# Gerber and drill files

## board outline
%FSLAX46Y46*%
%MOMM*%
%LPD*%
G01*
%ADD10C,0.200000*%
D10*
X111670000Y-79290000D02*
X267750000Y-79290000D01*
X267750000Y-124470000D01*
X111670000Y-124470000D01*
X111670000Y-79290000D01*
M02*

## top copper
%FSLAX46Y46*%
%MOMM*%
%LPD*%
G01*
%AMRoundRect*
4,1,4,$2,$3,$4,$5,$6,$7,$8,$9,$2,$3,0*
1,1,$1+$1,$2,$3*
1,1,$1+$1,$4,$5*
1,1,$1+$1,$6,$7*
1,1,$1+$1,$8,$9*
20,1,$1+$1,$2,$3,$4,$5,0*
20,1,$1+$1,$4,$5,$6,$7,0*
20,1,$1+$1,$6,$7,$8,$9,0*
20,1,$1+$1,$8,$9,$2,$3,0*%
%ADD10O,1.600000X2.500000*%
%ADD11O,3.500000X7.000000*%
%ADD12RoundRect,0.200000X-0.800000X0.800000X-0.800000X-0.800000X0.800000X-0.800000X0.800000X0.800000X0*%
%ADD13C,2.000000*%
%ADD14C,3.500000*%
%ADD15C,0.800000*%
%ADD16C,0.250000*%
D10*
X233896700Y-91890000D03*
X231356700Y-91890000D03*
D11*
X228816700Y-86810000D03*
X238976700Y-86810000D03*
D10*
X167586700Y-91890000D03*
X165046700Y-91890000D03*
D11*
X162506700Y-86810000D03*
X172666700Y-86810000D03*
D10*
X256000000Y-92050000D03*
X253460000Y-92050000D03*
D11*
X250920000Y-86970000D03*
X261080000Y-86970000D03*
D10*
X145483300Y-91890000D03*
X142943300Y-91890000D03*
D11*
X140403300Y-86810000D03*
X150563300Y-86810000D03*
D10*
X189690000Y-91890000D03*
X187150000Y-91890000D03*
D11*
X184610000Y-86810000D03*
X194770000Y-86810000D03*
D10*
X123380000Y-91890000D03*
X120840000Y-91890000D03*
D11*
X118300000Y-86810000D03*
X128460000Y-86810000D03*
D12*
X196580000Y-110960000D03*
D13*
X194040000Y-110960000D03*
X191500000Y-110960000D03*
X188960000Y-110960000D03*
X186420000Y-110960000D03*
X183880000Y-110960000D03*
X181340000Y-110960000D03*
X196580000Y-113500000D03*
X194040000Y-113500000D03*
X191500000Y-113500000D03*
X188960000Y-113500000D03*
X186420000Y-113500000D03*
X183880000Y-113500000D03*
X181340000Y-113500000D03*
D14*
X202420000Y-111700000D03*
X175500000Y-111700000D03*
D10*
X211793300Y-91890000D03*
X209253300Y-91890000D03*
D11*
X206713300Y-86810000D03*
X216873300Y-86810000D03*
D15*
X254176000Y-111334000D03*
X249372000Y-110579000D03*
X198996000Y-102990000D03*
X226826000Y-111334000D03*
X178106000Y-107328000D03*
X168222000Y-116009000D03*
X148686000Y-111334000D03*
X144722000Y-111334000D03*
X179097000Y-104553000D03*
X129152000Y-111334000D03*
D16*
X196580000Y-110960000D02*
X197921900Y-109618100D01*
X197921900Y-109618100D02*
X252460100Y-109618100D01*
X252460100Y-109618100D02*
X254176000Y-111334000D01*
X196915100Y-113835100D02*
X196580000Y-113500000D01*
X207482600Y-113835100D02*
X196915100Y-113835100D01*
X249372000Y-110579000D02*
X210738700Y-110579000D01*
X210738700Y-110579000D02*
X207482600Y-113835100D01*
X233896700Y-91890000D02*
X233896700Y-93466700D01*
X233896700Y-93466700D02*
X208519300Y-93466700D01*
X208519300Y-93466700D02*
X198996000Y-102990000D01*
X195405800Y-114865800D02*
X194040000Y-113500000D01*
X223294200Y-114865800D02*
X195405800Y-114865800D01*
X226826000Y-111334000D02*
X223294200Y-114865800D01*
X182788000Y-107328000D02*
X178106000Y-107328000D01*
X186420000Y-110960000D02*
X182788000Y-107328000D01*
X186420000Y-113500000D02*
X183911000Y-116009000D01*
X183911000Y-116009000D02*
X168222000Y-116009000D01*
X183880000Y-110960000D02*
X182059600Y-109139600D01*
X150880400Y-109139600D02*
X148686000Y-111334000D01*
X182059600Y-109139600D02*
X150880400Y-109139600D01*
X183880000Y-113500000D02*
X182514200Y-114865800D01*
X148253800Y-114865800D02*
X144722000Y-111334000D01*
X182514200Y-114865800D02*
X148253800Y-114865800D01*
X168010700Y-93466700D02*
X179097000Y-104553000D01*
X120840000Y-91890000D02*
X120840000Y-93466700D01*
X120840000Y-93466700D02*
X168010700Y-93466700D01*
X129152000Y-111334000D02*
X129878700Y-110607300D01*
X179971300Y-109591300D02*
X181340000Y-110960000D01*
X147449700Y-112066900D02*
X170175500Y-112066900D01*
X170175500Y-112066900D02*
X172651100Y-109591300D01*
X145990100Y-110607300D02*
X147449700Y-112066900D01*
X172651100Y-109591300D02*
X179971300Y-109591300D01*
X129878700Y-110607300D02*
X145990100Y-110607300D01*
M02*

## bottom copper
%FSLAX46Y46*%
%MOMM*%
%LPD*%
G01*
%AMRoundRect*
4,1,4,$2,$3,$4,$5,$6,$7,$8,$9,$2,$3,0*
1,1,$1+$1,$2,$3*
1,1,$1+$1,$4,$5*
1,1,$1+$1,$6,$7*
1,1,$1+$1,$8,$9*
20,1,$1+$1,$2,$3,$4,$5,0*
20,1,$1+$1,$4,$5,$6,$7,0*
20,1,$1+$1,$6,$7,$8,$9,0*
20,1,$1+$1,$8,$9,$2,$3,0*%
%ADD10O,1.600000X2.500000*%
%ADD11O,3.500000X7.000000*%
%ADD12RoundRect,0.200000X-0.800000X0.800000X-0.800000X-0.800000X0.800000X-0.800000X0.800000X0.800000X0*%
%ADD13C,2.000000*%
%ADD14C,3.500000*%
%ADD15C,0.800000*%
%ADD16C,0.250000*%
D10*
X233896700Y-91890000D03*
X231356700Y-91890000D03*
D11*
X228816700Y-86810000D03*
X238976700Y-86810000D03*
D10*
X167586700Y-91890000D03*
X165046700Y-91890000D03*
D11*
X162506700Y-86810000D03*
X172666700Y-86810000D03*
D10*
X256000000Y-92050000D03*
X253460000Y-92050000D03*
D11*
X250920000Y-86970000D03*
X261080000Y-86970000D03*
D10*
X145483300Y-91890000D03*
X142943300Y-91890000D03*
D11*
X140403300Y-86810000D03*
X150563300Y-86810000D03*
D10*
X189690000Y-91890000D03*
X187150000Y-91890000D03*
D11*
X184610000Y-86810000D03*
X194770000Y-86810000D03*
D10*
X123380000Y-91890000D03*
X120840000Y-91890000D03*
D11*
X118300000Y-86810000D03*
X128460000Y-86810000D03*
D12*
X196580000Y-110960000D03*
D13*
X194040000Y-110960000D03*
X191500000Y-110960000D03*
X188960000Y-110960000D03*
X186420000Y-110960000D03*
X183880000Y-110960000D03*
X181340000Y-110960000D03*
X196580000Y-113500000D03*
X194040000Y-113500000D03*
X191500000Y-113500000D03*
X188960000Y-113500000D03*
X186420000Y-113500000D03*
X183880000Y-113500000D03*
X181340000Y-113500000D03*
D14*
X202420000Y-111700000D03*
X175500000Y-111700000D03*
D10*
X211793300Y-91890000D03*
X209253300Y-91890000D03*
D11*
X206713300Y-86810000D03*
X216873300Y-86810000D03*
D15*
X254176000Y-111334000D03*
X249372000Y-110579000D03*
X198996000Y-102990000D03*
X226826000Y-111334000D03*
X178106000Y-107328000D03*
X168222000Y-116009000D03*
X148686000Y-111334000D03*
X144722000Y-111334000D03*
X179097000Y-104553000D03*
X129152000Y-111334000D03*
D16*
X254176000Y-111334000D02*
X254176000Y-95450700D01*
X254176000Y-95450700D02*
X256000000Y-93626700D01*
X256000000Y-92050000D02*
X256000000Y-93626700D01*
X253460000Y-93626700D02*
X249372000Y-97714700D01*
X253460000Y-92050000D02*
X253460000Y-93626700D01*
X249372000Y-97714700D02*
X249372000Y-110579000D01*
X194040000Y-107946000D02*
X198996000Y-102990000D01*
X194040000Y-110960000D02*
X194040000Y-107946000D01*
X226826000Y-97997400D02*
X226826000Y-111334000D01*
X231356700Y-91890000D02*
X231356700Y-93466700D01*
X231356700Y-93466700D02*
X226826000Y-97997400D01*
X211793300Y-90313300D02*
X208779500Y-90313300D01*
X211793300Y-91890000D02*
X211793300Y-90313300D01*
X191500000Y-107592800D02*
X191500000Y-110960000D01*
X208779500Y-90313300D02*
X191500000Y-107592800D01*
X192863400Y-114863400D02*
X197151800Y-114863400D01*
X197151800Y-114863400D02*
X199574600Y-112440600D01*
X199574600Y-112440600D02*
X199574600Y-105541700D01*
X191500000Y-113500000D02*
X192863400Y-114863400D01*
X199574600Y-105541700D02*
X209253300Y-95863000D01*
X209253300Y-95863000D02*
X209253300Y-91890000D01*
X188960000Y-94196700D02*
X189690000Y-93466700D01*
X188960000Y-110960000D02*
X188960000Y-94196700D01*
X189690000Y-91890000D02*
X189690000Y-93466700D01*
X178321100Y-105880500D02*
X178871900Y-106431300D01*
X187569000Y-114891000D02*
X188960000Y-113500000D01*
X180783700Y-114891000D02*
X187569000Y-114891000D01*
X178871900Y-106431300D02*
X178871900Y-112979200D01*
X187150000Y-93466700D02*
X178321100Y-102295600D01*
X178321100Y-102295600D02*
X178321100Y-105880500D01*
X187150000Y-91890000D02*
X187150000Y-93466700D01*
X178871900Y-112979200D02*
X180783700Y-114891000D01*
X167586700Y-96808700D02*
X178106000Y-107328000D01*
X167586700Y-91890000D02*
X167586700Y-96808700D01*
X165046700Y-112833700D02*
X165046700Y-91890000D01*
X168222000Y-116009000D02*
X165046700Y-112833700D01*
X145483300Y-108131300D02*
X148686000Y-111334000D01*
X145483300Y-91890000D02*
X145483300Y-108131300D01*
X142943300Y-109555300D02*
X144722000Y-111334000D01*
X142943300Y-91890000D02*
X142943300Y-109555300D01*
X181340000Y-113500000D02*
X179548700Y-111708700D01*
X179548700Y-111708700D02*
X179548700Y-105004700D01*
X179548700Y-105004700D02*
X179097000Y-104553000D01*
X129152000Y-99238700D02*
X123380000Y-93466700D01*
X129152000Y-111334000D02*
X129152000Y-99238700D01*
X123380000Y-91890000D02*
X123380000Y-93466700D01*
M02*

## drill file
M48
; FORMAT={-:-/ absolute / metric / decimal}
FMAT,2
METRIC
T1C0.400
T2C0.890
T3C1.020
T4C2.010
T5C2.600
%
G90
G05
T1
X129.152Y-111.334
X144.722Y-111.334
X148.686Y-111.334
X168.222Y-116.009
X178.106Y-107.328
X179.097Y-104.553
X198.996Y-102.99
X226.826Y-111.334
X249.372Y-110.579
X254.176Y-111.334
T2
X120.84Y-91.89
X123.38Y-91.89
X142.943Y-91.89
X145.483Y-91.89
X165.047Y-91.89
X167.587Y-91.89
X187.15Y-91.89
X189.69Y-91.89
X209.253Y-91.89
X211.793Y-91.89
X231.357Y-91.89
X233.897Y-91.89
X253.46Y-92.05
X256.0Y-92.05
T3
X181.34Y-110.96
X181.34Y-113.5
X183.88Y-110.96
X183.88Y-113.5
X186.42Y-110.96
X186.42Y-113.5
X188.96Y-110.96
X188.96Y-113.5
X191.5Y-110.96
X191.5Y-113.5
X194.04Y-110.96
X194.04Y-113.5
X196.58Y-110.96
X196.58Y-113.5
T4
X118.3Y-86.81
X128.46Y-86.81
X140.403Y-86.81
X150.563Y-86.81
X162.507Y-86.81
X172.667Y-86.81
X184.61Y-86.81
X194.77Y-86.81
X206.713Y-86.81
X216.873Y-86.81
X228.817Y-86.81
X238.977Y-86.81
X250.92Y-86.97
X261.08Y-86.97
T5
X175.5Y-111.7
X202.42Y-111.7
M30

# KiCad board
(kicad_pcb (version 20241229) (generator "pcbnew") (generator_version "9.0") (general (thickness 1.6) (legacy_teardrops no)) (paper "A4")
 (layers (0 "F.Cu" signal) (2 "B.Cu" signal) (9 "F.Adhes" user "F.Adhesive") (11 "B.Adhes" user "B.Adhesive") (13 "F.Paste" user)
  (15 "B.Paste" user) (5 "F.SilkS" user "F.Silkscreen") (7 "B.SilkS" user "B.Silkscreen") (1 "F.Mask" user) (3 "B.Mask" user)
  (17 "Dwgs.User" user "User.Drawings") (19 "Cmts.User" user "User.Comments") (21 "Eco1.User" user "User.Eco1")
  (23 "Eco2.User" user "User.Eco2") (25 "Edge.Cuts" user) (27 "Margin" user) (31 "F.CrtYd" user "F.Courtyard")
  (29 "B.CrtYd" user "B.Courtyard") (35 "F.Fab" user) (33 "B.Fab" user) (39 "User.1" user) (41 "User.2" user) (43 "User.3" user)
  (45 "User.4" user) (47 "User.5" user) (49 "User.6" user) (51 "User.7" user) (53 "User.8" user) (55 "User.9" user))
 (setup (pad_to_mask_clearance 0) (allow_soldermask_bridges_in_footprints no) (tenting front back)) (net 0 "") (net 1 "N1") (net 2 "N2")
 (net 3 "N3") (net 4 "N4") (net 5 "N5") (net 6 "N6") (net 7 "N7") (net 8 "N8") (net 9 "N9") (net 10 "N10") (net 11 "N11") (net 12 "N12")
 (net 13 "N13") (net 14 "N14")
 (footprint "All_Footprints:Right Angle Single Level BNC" (layer "F.Cu") (at 233.8967 91.89)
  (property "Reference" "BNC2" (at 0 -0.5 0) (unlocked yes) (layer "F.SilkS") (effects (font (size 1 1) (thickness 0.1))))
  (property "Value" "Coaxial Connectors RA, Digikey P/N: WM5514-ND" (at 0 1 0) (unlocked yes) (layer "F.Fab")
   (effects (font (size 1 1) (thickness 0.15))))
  (pad "1" thru_hole oval (at 0 0) (size 1.6 2.5) (drill 0.89) (layers "*.Cu" "*.Mask") (remove_unused_layers no) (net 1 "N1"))
  (pad "2" thru_hole oval (at -2.54 0) (size 1.6 2.5) (drill 0.89) (layers "*.Cu" "*.Mask") (remove_unused_layers no) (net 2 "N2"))
  (pad "MH" thru_hole oval (at -5.08 -5.08) (size 3.5 7) (drill 2.01) (layers "*.Cu" "*.Mask") (remove_unused_layers no))
  (pad "MH" thru_hole oval (at 5.08 -5.08) (size 3.5 7) (drill 2.01) (layers "*.Cu" "*.Mask") (remove_unused_layers no)))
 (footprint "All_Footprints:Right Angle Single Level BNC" (layer "F.Cu") (at 167.5867 91.89)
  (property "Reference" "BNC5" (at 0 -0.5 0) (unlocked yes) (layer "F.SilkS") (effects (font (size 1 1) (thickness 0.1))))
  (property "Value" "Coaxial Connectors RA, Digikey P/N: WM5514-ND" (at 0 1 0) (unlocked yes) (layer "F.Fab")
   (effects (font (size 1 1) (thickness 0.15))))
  (pad "1" thru_hole oval (at 0 0) (size 1.6 2.5) (drill 0.89) (layers "*.Cu" "*.Mask") (remove_unused_layers no) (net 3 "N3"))
  (pad "2" thru_hole oval (at -2.54 0) (size 1.6 2.5) (drill 0.89) (layers "*.Cu" "*.Mask") (remove_unused_layers no) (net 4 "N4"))
  (pad "MH" thru_hole oval (at -5.08 -5.08) (size 3.5 7) (drill 2.01) (layers "*.Cu" "*.Mask") (remove_unused_layers no))
  (pad "MH" thru_hole oval (at 5.08 -5.08) (size 3.5 7) (drill 2.01) (layers "*.Cu" "*.Mask") (remove_unused_layers no)))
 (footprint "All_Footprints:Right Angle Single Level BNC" (layer "F.Cu") (at 256 92.05)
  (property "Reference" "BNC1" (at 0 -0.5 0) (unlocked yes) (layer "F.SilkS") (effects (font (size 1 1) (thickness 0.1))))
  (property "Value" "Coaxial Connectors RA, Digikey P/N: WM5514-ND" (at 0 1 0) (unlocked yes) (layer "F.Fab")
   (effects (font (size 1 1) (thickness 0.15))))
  (pad "1" thru_hole oval (at 0 0) (size 1.6 2.5) (drill 0.89) (layers "*.Cu" "*.Mask") (remove_unused_layers no) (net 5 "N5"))
  (pad "2" thru_hole oval (at -2.54 0) (size 1.6 2.5) (drill 0.89) (layers "*.Cu" "*.Mask") (remove_unused_layers no) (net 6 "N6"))
  (pad "MH" thru_hole oval (at -5.08 -5.08) (size 3.5 7) (drill 2.01) (layers "*.Cu" "*.Mask") (remove_unused_layers no))
  (pad "MH" thru_hole oval (at 5.08 -5.08) (size 3.5 7) (drill 2.01) (layers "*.Cu" "*.Mask") (remove_unused_layers no)))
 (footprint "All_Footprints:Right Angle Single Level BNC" (layer "F.Cu") (at 145.4833 91.89)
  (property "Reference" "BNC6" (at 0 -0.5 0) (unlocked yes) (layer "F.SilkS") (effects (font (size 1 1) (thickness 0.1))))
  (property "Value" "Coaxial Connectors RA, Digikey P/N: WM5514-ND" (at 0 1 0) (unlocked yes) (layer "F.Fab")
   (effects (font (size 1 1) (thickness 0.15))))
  (pad "1" thru_hole oval (at 0 0) (size 1.6 2.5) (drill 0.89) (layers "*.Cu" "*.Mask") (remove_unused_layers no) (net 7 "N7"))
  (pad "2" thru_hole oval (at -2.54 0) (size 1.6 2.5) (drill 0.89) (layers "*.Cu" "*.Mask") (remove_unused_layers no) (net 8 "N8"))
  (pad "MH" thru_hole oval (at -5.08 -5.08) (size 3.5 7) (drill 2.01) (layers "*.Cu" "*.Mask") (remove_unused_layers no))
  (pad "MH" thru_hole oval (at 5.08 -5.08) (size 3.5 7) (drill 2.01) (layers "*.Cu" "*.Mask") (remove_unused_layers no)))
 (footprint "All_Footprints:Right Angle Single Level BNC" (layer "F.Cu") (at 189.69 91.89)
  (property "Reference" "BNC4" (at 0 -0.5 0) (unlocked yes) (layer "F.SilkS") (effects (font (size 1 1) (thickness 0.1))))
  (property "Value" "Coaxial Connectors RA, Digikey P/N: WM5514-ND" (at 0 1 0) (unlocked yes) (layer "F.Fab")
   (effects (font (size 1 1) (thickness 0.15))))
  (pad "1" thru_hole oval (at 0 0) (size 1.6 2.5) (drill 0.89) (layers "*.Cu" "*.Mask") (remove_unused_layers no) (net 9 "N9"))
  (pad "2" thru_hole oval (at -2.54 0) (size 1.6 2.5) (drill 0.89) (layers "*.Cu" "*.Mask") (remove_unused_layers no) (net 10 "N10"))
  (pad "MH" thru_hole oval (at -5.08 -5.08) (size 3.5 7) (drill 2.01) (layers "*.Cu" "*.Mask") (remove_unused_layers no))
  (pad "MH" thru_hole oval (at 5.08 -5.08) (size 3.5 7) (drill 2.01) (layers "*.Cu" "*.Mask") (remove_unused_layers no)))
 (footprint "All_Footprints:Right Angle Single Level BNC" (layer "F.Cu") (at 123.38 91.89)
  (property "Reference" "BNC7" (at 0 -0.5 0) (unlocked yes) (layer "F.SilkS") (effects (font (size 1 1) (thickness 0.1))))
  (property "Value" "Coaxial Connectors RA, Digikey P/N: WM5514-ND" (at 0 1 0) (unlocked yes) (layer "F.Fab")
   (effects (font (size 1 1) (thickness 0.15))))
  (pad "1" thru_hole oval (at 0 0) (size 1.6 2.5) (drill 0.89) (layers "*.Cu" "*.Mask") (remove_unused_layers no) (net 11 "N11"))
  (pad "2" thru_hole oval (at -2.54 0) (size 1.6 2.5) (drill 0.89) (layers "*.Cu" "*.Mask") (remove_unused_layers no) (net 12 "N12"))
  (pad "MH" thru_hole oval (at -5.08 -5.08) (size 3.5 7) (drill 2.01) (layers "*.Cu" "*.Mask") (remove_unused_layers no))
  (pad "MH" thru_hole oval (at 5.08 -5.08) (size 3.5 7) (drill 2.01) (layers "*.Cu" "*.Mask") (remove_unused_layers no)))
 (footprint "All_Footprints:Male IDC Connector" (layer "F.Cu") (at 207.42 105.85 -90)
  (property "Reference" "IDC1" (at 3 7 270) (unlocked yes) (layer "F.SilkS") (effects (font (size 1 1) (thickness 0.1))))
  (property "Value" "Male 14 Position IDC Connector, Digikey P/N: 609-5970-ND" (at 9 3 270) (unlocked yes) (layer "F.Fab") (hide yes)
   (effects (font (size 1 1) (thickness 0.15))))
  (pad "1" thru_hole roundrect (at 5.11 10.84 270) (size 2 2) (drill 1.02) (layers "*.Cu" "*.Mask") (remove_unused_layers no)
   (roundrect_rratio 0.1) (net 5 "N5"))
  (pad "2" thru_hole circle (at 5.11 13.38 270) (size 2 2) (drill 1.02) (layers "*.Cu" "*.Mask") (remove_unused_layers no) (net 1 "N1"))
  (pad "3" thru_hole circle (at 5.11 15.92 270) (size 2 2) (drill 1.02) (layers "*.Cu" "*.Mask") (remove_unused_layers no) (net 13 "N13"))
  (pad "4" thru_hole circle (at 5.11 18.46 270) (size 2 2) (drill 1.02) (layers "*.Cu" "*.Mask") (remove_unused_layers no) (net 9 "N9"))
  (pad "5" thru_hole circle (at 5.11 21 270) (size 2 2) (drill 1.02) (layers "*.Cu" "*.Mask") (remove_unused_layers no) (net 3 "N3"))
  (pad "6" thru_hole circle (at 5.11 23.54 270) (size 2 2) (drill 1.02) (layers "*.Cu" "*.Mask") (remove_unused_layers no) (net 7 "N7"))
  (pad "7" thru_hole circle (at 5.11 26.08 270) (size 2 2) (drill 1.02) (layers "*.Cu" "*.Mask") (remove_unused_layers no) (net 11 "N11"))
  (pad "8" thru_hole circle (at 7.65 10.84 270) (size 2 2) (drill 1.02) (layers "*.Cu" "*.Mask") (remove_unused_layers no) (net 6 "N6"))
  (pad "9" thru_hole circle (at 7.65 13.38 270) (size 2 2) (drill 1.02) (layers "*.Cu" "*.Mask") (remove_unused_layers no) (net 2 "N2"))
  (pad "10" thru_hole circle (at 7.65 15.92 270) (size 2 2) (drill 1.02) (layers "*.Cu" "*.Mask") (remove_unused_layers no) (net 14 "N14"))
  (pad "11" thru_hole circle (at 7.65 18.46 270) (size 2 2) (drill 1.02) (layers "*.Cu" "*.Mask") (remove_unused_layers no) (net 10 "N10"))
  (pad "12" thru_hole circle (at 7.65 21 270) (size 2 2) (drill 1.02) (layers "*.Cu" "*.Mask") (remove_unused_layers no) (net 4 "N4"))
  (pad "13" thru_hole circle (at 7.65 23.54 270) (size 2 2) (drill 1.02) (layers "*.Cu" "*.Mask") (remove_unused_layers no) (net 8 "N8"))
  (pad "14" thru_hole circle (at 7.65 26.08 270) (size 2 2) (drill 1.02) (layers "*.Cu" "*.Mask") (remove_unused_layers no) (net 12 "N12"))
  (pad "MH" thru_hole circle (at 5.85 5 270) (size 3.5 3.5) (drill 2.6) (layers "*.Cu" "*.Mask") (remove_unused_layers no))
  (pad "MH" thru_hole circle (at 5.85 31.92 270) (size 3.5 3.5) (drill 2.6) (layers "*.Cu" "*.Mask") (remove_unused_layers no)))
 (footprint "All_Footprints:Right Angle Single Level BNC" (layer "F.Cu") (at 211.7933 91.89)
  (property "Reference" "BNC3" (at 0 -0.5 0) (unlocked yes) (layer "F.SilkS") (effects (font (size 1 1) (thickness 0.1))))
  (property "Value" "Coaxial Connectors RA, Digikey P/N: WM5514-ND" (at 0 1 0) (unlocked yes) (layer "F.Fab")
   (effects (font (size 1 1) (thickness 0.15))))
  (pad "1" thru_hole oval (at 0 0) (size 1.6 2.5) (drill 0.89) (layers "*.Cu" "*.Mask") (remove_unused_layers no) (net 13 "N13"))
  (pad "2" thru_hole oval (at -2.54 0) (size 1.6 2.5) (drill 0.89) (layers "*.Cu" "*.Mask") (remove_unused_layers no) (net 14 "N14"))
  (pad "MH" thru_hole oval (at -5.08 -5.08) (size 3.5 7) (drill 2.01) (layers "*.Cu" "*.Mask") (remove_unused_layers no))
  (pad "MH" thru_hole oval (at 5.08 -5.08) (size 3.5 7) (drill 2.01) (layers "*.Cu" "*.Mask") (remove_unused_layers no)))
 (gr_rect (start 111.67 79.29) (end 267.75 124.47) (stroke (width 0.2) (type solid)) (fill no) (layer "Edge.Cuts"))
 (segment (start 196.58 110.96) (end 197.9219 109.6181) (width 0.25) (layer "F.Cu") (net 5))
 (segment (start 197.9219 109.6181) (end 252.4601 109.6181) (width 0.25) (layer "F.Cu") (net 5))
 (segment (start 252.4601 109.6181) (end 254.176 111.334) (width 0.25) (layer "F.Cu") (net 5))
 (via (at 254.176 111.334) (size 0.8) (drill 0.4) (layers "F.Cu" "B.Cu") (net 5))
 (segment (start 254.176 111.334) (end 254.176 95.4507) (width 0.25) (layer "B.Cu") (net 5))
 (segment (start 254.176 95.4507) (end 256 93.6267) (width 0.25) (layer "B.Cu") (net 5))
 (segment (start 256 92.05) (end 256 93.6267) (width 0.25) (layer "B.Cu") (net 5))
 (segment (start 196.9151 113.8351) (end 196.58 113.5) (width 0.25) (layer "F.Cu") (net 6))
 (segment (start 207.4826 113.8351) (end 196.9151 113.8351) (width 0.25) (layer "F.Cu") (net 6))
 (segment (start 249.372 110.579) (end 210.7387 110.579) (width 0.25) (layer "F.Cu") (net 6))
 (segment (start 210.7387 110.579) (end 207.4826 113.8351) (width 0.25) (layer "F.Cu") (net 6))
 (via (at 249.372 110.579) (size 0.8) (drill 0.4) (layers "F.Cu" "B.Cu") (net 6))
 (segment (start 253.46 93.6267) (end 249.372 97.7147) (width 0.25) (layer "B.Cu") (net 6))
 (segment (start 253.46 92.05) (end 253.46 93.6267) (width 0.25) (layer "B.Cu") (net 6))
 (segment (start 249.372 97.7147) (end 249.372 110.579) (width 0.25) (layer "B.Cu") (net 6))
 (segment (start 233.8967 91.89) (end 233.8967 93.4667) (width 0.25) (layer "F.Cu") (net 1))
 (segment (start 233.8967 93.4667) (end 208.5193 93.4667) (width 0.25) (layer "F.Cu") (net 1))
 (segment (start 208.5193 93.4667) (end 198.996 102.99) (width 0.25) (layer "F.Cu") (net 1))
 (via (at 198.996 102.99) (size 0.8) (drill 0.4) (layers "F.Cu" "B.Cu") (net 1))
 (segment (start 194.04 107.946) (end 198.996 102.99) (width 0.25) (layer "B.Cu") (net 1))
 (segment (start 194.04 110.96) (end 194.04 107.946) (width 0.25) (layer "B.Cu") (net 1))
 (segment (start 195.4058 114.8658) (end 194.04 113.5) (width 0.25) (layer "F.Cu") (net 2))
 (segment (start 223.2942 114.8658) (end 195.4058 114.8658) (width 0.25) (layer "F.Cu") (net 2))
 (segment (start 226.826 111.334) (end 223.2942 114.8658) (width 0.25) (layer "F.Cu") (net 2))
 (via (at 226.826 111.334) (size 0.8) (drill 0.4) (layers "F.Cu" "B.Cu") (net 2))
 (segment (start 226.826 97.9974) (end 226.826 111.334) (width 0.25) (layer "B.Cu") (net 2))
 (segment (start 231.3567 91.89) (end 231.3567 93.4667) (width 0.25) (layer "B.Cu") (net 2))
 (segment (start 231.3567 93.4667) (end 226.826 97.9974) (width 0.25) (layer "B.Cu") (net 2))
 (segment (start 211.7933 90.3133) (end 208.7795 90.3133) (width 0.25) (layer "B.Cu") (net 13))
 (segment (start 211.7933 91.89) (end 211.7933 90.3133) (width 0.25) (layer "B.Cu") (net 13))
 (segment (start 191.5 107.5928) (end 191.5 110.96) (width 0.25) (layer "B.Cu") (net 13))
 (segment (start 208.7795 90.3133) (end 191.5 107.5928) (width 0.25) (layer "B.Cu") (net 13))
 (segment (start 192.8634 114.8634) (end 197.1518 114.8634) (width 0.25) (layer "B.Cu") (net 14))
 (segment (start 197.1518 114.8634) (end 199.5746 112.4406) (width 0.25) (layer "B.Cu") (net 14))
 (segment (start 199.5746 112.4406) (end 199.5746 105.5417) (width 0.25) (layer "B.Cu") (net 14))
 (segment (start 191.5 113.5) (end 192.8634 114.8634) (width 0.25) (layer "B.Cu") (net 14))
 (segment (start 199.5746 105.5417) (end 209.2533 95.863) (width 0.25) (layer "B.Cu") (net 14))
 (segment (start 209.2533 95.863) (end 209.2533 91.89) (width 0.25) (layer "B.Cu") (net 14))
 (segment (start 188.96 94.1967) (end 189.69 93.4667) (width 0.25) (layer "B.Cu") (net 9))
 (segment (start 188.96 110.96) (end 188.96 94.1967) (width 0.25) (layer "B.Cu") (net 9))
 (segment (start 189.69 91.89) (end 189.69 93.4667) (width 0.25) (layer "B.Cu") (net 9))
 (segment (start 178.3211 105.8805) (end 178.8719 106.4313) (width 0.25) (layer "B.Cu") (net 10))
 (segment (start 187.569 114.891) (end 188.96 113.5) (width 0.25) (layer "B.Cu") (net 10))
 (segment (start 180.7837 114.891) (end 187.569 114.891) (width 0.25) (layer "B.Cu") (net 10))
 (segment (start 178.8719 106.4313) (end 178.8719 112.9792) (width 0.25) (layer "B.Cu") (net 10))
 (segment (start 187.15 93.4667) (end 178.3211 102.2956) (width 0.25) (layer "B.Cu") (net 10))
 (segment (start 178.3211 102.2956) (end 178.3211 105.8805) (width 0.25) (layer "B.Cu") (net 10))
 (segment (start 187.15 91.89) (end 187.15 93.4667) (width 0.25) (layer "B.Cu") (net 10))
 (segment (start 178.8719 112.9792) (end 180.7837 114.891) (width 0.25) (layer "B.Cu") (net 10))
 (segment (start 182.788 107.328) (end 178.106 107.328) (width 0.25) (layer "F.Cu") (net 3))
 (segment (start 186.42 110.96) (end 182.788 107.328) (width 0.25) (layer "F.Cu") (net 3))
 (via (at 178.106 107.328) (size 0.8) (drill 0.4) (layers "F.Cu" "B.Cu") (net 3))
 (segment (start 167.5867 96.8087) (end 178.106 107.328) (width 0.25) (layer "B.Cu") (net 3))
 (segment (start 167.5867 91.89) (end 167.5867 96.8087) (width 0.25) (layer "B.Cu") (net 3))
 (segment (start 186.42 113.5) (end 183.911 116.009) (width 0.25) (layer "F.Cu") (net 4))
 (segment (start 183.911 116.009) (end 168.222 116.009) (width 0.25) (layer "F.Cu") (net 4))
 (via (at 168.222 116.009) (size 0.8) (drill 0.4) (layers "F.Cu" "B.Cu") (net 4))
 (segment (start 165.0467 112.8337) (end 165.0467 91.89) (width 0.25) (layer "B.Cu") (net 4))
 (segment (start 168.222 116.009) (end 165.0467 112.8337) (width 0.25) (layer "B.Cu") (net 4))
 (segment (start 183.88 110.96) (end 182.0596 109.1396) (width 0.25) (layer "F.Cu") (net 7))
 (segment (start 150.8804 109.1396) (end 148.686 111.334) (width 0.25) (layer "F.Cu") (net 7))
 (segment (start 182.0596 109.1396) (end 150.8804 109.1396) (width 0.25) (layer "F.Cu") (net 7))
 (via (at 148.686 111.334) (size 0.8) (drill 0.4) (layers "F.Cu" "B.Cu") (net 7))
 (segment (start 145.4833 108.1313) (end 148.686 111.334) (width 0.25) (layer "B.Cu") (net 7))
 (segment (start 145.4833 91.89) (end 145.4833 108.1313) (width 0.25) (layer "B.Cu") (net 7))
 (segment (start 183.88 113.5) (end 182.5142 114.8658) (width 0.25) (layer "F.Cu") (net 8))
 (segment (start 148.2538 114.8658) (end 144.722 111.334) (width 0.25) (layer "F.Cu") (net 8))
 (segment (start 182.5142 114.8658) (end 148.2538 114.8658) (width 0.25) (layer "F.Cu") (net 8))
 (via (at 144.722 111.334) (size 0.8) (drill 0.4) (layers "F.Cu" "B.Cu") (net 8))
 (segment (start 142.9433 109.5553) (end 144.722 111.334) (width 0.25) (layer "B.Cu") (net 8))
 (segment (start 142.9433 91.89) (end 142.9433 109.5553) (width 0.25) (layer "B.Cu") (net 8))
 (segment (start 168.0107 93.4667) (end 179.097 104.553) (width 0.25) (layer "F.Cu") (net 12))
 (segment (start 120.84 91.89) (end 120.84 93.4667) (width 0.25) (layer "F.Cu") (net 12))
 (segment (start 120.84 93.4667) (end 168.0107 93.4667) (width 0.25) (layer "F.Cu") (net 12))
 (via (at 179.097 104.553) (size 0.8) (drill 0.4) (layers "F.Cu" "B.Cu") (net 12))
 (segment (start 181.34 113.5) (end 179.5487 111.7087) (width 0.25) (layer "B.Cu") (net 12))
 (segment (start 179.5487 111.7087) (end 179.5487 105.0047) (width 0.25) (layer "B.Cu") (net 12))
 (segment (start 179.5487 105.0047) (end 179.097 104.553) (width 0.25) (layer "B.Cu") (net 12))
 (segment (start 129.152 111.334) (end 129.8787 110.6073) (width 0.25) (layer "F.Cu") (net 11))
 (segment (start 179.9713 109.5913) (end 181.34 110.96) (width 0.25) (layer "F.Cu") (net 11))
 (segment (start 147.4497 112.0669) (end 170.1755 112.0669) (width 0.25) (layer "F.Cu") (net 11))
 (segment (start 170.1755 112.0669) (end 172.6511 109.5913) (width 0.25) (layer "F.Cu") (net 11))
 (segment (start 145.9901 110.6073) (end 147.4497 112.0669) (width 0.25) (layer "F.Cu") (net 11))
 (segment (start 172.6511 109.5913) (end 179.9713 109.5913) (width 0.25) (layer "F.Cu") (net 11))
 (segment (start 129.8787 110.6073) (end 145.9901 110.6073) (width 0.25) (layer "F.Cu") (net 11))
 (via (at 129.152 111.334) (size 0.8) (drill 0.4) (layers "F.Cu" "B.Cu") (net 11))
 (segment (start 129.152 99.2387) (end 123.38 93.4667) (width 0.25) (layer "B.Cu") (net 11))
 (segment (start 129.152 111.334) (end 129.152 99.2387) (width 0.25) (layer "B.Cu") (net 11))
 (segment (start 123.38 91.89) (end 123.38 93.4667) (width 0.25) (layer "B.Cu") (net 11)))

